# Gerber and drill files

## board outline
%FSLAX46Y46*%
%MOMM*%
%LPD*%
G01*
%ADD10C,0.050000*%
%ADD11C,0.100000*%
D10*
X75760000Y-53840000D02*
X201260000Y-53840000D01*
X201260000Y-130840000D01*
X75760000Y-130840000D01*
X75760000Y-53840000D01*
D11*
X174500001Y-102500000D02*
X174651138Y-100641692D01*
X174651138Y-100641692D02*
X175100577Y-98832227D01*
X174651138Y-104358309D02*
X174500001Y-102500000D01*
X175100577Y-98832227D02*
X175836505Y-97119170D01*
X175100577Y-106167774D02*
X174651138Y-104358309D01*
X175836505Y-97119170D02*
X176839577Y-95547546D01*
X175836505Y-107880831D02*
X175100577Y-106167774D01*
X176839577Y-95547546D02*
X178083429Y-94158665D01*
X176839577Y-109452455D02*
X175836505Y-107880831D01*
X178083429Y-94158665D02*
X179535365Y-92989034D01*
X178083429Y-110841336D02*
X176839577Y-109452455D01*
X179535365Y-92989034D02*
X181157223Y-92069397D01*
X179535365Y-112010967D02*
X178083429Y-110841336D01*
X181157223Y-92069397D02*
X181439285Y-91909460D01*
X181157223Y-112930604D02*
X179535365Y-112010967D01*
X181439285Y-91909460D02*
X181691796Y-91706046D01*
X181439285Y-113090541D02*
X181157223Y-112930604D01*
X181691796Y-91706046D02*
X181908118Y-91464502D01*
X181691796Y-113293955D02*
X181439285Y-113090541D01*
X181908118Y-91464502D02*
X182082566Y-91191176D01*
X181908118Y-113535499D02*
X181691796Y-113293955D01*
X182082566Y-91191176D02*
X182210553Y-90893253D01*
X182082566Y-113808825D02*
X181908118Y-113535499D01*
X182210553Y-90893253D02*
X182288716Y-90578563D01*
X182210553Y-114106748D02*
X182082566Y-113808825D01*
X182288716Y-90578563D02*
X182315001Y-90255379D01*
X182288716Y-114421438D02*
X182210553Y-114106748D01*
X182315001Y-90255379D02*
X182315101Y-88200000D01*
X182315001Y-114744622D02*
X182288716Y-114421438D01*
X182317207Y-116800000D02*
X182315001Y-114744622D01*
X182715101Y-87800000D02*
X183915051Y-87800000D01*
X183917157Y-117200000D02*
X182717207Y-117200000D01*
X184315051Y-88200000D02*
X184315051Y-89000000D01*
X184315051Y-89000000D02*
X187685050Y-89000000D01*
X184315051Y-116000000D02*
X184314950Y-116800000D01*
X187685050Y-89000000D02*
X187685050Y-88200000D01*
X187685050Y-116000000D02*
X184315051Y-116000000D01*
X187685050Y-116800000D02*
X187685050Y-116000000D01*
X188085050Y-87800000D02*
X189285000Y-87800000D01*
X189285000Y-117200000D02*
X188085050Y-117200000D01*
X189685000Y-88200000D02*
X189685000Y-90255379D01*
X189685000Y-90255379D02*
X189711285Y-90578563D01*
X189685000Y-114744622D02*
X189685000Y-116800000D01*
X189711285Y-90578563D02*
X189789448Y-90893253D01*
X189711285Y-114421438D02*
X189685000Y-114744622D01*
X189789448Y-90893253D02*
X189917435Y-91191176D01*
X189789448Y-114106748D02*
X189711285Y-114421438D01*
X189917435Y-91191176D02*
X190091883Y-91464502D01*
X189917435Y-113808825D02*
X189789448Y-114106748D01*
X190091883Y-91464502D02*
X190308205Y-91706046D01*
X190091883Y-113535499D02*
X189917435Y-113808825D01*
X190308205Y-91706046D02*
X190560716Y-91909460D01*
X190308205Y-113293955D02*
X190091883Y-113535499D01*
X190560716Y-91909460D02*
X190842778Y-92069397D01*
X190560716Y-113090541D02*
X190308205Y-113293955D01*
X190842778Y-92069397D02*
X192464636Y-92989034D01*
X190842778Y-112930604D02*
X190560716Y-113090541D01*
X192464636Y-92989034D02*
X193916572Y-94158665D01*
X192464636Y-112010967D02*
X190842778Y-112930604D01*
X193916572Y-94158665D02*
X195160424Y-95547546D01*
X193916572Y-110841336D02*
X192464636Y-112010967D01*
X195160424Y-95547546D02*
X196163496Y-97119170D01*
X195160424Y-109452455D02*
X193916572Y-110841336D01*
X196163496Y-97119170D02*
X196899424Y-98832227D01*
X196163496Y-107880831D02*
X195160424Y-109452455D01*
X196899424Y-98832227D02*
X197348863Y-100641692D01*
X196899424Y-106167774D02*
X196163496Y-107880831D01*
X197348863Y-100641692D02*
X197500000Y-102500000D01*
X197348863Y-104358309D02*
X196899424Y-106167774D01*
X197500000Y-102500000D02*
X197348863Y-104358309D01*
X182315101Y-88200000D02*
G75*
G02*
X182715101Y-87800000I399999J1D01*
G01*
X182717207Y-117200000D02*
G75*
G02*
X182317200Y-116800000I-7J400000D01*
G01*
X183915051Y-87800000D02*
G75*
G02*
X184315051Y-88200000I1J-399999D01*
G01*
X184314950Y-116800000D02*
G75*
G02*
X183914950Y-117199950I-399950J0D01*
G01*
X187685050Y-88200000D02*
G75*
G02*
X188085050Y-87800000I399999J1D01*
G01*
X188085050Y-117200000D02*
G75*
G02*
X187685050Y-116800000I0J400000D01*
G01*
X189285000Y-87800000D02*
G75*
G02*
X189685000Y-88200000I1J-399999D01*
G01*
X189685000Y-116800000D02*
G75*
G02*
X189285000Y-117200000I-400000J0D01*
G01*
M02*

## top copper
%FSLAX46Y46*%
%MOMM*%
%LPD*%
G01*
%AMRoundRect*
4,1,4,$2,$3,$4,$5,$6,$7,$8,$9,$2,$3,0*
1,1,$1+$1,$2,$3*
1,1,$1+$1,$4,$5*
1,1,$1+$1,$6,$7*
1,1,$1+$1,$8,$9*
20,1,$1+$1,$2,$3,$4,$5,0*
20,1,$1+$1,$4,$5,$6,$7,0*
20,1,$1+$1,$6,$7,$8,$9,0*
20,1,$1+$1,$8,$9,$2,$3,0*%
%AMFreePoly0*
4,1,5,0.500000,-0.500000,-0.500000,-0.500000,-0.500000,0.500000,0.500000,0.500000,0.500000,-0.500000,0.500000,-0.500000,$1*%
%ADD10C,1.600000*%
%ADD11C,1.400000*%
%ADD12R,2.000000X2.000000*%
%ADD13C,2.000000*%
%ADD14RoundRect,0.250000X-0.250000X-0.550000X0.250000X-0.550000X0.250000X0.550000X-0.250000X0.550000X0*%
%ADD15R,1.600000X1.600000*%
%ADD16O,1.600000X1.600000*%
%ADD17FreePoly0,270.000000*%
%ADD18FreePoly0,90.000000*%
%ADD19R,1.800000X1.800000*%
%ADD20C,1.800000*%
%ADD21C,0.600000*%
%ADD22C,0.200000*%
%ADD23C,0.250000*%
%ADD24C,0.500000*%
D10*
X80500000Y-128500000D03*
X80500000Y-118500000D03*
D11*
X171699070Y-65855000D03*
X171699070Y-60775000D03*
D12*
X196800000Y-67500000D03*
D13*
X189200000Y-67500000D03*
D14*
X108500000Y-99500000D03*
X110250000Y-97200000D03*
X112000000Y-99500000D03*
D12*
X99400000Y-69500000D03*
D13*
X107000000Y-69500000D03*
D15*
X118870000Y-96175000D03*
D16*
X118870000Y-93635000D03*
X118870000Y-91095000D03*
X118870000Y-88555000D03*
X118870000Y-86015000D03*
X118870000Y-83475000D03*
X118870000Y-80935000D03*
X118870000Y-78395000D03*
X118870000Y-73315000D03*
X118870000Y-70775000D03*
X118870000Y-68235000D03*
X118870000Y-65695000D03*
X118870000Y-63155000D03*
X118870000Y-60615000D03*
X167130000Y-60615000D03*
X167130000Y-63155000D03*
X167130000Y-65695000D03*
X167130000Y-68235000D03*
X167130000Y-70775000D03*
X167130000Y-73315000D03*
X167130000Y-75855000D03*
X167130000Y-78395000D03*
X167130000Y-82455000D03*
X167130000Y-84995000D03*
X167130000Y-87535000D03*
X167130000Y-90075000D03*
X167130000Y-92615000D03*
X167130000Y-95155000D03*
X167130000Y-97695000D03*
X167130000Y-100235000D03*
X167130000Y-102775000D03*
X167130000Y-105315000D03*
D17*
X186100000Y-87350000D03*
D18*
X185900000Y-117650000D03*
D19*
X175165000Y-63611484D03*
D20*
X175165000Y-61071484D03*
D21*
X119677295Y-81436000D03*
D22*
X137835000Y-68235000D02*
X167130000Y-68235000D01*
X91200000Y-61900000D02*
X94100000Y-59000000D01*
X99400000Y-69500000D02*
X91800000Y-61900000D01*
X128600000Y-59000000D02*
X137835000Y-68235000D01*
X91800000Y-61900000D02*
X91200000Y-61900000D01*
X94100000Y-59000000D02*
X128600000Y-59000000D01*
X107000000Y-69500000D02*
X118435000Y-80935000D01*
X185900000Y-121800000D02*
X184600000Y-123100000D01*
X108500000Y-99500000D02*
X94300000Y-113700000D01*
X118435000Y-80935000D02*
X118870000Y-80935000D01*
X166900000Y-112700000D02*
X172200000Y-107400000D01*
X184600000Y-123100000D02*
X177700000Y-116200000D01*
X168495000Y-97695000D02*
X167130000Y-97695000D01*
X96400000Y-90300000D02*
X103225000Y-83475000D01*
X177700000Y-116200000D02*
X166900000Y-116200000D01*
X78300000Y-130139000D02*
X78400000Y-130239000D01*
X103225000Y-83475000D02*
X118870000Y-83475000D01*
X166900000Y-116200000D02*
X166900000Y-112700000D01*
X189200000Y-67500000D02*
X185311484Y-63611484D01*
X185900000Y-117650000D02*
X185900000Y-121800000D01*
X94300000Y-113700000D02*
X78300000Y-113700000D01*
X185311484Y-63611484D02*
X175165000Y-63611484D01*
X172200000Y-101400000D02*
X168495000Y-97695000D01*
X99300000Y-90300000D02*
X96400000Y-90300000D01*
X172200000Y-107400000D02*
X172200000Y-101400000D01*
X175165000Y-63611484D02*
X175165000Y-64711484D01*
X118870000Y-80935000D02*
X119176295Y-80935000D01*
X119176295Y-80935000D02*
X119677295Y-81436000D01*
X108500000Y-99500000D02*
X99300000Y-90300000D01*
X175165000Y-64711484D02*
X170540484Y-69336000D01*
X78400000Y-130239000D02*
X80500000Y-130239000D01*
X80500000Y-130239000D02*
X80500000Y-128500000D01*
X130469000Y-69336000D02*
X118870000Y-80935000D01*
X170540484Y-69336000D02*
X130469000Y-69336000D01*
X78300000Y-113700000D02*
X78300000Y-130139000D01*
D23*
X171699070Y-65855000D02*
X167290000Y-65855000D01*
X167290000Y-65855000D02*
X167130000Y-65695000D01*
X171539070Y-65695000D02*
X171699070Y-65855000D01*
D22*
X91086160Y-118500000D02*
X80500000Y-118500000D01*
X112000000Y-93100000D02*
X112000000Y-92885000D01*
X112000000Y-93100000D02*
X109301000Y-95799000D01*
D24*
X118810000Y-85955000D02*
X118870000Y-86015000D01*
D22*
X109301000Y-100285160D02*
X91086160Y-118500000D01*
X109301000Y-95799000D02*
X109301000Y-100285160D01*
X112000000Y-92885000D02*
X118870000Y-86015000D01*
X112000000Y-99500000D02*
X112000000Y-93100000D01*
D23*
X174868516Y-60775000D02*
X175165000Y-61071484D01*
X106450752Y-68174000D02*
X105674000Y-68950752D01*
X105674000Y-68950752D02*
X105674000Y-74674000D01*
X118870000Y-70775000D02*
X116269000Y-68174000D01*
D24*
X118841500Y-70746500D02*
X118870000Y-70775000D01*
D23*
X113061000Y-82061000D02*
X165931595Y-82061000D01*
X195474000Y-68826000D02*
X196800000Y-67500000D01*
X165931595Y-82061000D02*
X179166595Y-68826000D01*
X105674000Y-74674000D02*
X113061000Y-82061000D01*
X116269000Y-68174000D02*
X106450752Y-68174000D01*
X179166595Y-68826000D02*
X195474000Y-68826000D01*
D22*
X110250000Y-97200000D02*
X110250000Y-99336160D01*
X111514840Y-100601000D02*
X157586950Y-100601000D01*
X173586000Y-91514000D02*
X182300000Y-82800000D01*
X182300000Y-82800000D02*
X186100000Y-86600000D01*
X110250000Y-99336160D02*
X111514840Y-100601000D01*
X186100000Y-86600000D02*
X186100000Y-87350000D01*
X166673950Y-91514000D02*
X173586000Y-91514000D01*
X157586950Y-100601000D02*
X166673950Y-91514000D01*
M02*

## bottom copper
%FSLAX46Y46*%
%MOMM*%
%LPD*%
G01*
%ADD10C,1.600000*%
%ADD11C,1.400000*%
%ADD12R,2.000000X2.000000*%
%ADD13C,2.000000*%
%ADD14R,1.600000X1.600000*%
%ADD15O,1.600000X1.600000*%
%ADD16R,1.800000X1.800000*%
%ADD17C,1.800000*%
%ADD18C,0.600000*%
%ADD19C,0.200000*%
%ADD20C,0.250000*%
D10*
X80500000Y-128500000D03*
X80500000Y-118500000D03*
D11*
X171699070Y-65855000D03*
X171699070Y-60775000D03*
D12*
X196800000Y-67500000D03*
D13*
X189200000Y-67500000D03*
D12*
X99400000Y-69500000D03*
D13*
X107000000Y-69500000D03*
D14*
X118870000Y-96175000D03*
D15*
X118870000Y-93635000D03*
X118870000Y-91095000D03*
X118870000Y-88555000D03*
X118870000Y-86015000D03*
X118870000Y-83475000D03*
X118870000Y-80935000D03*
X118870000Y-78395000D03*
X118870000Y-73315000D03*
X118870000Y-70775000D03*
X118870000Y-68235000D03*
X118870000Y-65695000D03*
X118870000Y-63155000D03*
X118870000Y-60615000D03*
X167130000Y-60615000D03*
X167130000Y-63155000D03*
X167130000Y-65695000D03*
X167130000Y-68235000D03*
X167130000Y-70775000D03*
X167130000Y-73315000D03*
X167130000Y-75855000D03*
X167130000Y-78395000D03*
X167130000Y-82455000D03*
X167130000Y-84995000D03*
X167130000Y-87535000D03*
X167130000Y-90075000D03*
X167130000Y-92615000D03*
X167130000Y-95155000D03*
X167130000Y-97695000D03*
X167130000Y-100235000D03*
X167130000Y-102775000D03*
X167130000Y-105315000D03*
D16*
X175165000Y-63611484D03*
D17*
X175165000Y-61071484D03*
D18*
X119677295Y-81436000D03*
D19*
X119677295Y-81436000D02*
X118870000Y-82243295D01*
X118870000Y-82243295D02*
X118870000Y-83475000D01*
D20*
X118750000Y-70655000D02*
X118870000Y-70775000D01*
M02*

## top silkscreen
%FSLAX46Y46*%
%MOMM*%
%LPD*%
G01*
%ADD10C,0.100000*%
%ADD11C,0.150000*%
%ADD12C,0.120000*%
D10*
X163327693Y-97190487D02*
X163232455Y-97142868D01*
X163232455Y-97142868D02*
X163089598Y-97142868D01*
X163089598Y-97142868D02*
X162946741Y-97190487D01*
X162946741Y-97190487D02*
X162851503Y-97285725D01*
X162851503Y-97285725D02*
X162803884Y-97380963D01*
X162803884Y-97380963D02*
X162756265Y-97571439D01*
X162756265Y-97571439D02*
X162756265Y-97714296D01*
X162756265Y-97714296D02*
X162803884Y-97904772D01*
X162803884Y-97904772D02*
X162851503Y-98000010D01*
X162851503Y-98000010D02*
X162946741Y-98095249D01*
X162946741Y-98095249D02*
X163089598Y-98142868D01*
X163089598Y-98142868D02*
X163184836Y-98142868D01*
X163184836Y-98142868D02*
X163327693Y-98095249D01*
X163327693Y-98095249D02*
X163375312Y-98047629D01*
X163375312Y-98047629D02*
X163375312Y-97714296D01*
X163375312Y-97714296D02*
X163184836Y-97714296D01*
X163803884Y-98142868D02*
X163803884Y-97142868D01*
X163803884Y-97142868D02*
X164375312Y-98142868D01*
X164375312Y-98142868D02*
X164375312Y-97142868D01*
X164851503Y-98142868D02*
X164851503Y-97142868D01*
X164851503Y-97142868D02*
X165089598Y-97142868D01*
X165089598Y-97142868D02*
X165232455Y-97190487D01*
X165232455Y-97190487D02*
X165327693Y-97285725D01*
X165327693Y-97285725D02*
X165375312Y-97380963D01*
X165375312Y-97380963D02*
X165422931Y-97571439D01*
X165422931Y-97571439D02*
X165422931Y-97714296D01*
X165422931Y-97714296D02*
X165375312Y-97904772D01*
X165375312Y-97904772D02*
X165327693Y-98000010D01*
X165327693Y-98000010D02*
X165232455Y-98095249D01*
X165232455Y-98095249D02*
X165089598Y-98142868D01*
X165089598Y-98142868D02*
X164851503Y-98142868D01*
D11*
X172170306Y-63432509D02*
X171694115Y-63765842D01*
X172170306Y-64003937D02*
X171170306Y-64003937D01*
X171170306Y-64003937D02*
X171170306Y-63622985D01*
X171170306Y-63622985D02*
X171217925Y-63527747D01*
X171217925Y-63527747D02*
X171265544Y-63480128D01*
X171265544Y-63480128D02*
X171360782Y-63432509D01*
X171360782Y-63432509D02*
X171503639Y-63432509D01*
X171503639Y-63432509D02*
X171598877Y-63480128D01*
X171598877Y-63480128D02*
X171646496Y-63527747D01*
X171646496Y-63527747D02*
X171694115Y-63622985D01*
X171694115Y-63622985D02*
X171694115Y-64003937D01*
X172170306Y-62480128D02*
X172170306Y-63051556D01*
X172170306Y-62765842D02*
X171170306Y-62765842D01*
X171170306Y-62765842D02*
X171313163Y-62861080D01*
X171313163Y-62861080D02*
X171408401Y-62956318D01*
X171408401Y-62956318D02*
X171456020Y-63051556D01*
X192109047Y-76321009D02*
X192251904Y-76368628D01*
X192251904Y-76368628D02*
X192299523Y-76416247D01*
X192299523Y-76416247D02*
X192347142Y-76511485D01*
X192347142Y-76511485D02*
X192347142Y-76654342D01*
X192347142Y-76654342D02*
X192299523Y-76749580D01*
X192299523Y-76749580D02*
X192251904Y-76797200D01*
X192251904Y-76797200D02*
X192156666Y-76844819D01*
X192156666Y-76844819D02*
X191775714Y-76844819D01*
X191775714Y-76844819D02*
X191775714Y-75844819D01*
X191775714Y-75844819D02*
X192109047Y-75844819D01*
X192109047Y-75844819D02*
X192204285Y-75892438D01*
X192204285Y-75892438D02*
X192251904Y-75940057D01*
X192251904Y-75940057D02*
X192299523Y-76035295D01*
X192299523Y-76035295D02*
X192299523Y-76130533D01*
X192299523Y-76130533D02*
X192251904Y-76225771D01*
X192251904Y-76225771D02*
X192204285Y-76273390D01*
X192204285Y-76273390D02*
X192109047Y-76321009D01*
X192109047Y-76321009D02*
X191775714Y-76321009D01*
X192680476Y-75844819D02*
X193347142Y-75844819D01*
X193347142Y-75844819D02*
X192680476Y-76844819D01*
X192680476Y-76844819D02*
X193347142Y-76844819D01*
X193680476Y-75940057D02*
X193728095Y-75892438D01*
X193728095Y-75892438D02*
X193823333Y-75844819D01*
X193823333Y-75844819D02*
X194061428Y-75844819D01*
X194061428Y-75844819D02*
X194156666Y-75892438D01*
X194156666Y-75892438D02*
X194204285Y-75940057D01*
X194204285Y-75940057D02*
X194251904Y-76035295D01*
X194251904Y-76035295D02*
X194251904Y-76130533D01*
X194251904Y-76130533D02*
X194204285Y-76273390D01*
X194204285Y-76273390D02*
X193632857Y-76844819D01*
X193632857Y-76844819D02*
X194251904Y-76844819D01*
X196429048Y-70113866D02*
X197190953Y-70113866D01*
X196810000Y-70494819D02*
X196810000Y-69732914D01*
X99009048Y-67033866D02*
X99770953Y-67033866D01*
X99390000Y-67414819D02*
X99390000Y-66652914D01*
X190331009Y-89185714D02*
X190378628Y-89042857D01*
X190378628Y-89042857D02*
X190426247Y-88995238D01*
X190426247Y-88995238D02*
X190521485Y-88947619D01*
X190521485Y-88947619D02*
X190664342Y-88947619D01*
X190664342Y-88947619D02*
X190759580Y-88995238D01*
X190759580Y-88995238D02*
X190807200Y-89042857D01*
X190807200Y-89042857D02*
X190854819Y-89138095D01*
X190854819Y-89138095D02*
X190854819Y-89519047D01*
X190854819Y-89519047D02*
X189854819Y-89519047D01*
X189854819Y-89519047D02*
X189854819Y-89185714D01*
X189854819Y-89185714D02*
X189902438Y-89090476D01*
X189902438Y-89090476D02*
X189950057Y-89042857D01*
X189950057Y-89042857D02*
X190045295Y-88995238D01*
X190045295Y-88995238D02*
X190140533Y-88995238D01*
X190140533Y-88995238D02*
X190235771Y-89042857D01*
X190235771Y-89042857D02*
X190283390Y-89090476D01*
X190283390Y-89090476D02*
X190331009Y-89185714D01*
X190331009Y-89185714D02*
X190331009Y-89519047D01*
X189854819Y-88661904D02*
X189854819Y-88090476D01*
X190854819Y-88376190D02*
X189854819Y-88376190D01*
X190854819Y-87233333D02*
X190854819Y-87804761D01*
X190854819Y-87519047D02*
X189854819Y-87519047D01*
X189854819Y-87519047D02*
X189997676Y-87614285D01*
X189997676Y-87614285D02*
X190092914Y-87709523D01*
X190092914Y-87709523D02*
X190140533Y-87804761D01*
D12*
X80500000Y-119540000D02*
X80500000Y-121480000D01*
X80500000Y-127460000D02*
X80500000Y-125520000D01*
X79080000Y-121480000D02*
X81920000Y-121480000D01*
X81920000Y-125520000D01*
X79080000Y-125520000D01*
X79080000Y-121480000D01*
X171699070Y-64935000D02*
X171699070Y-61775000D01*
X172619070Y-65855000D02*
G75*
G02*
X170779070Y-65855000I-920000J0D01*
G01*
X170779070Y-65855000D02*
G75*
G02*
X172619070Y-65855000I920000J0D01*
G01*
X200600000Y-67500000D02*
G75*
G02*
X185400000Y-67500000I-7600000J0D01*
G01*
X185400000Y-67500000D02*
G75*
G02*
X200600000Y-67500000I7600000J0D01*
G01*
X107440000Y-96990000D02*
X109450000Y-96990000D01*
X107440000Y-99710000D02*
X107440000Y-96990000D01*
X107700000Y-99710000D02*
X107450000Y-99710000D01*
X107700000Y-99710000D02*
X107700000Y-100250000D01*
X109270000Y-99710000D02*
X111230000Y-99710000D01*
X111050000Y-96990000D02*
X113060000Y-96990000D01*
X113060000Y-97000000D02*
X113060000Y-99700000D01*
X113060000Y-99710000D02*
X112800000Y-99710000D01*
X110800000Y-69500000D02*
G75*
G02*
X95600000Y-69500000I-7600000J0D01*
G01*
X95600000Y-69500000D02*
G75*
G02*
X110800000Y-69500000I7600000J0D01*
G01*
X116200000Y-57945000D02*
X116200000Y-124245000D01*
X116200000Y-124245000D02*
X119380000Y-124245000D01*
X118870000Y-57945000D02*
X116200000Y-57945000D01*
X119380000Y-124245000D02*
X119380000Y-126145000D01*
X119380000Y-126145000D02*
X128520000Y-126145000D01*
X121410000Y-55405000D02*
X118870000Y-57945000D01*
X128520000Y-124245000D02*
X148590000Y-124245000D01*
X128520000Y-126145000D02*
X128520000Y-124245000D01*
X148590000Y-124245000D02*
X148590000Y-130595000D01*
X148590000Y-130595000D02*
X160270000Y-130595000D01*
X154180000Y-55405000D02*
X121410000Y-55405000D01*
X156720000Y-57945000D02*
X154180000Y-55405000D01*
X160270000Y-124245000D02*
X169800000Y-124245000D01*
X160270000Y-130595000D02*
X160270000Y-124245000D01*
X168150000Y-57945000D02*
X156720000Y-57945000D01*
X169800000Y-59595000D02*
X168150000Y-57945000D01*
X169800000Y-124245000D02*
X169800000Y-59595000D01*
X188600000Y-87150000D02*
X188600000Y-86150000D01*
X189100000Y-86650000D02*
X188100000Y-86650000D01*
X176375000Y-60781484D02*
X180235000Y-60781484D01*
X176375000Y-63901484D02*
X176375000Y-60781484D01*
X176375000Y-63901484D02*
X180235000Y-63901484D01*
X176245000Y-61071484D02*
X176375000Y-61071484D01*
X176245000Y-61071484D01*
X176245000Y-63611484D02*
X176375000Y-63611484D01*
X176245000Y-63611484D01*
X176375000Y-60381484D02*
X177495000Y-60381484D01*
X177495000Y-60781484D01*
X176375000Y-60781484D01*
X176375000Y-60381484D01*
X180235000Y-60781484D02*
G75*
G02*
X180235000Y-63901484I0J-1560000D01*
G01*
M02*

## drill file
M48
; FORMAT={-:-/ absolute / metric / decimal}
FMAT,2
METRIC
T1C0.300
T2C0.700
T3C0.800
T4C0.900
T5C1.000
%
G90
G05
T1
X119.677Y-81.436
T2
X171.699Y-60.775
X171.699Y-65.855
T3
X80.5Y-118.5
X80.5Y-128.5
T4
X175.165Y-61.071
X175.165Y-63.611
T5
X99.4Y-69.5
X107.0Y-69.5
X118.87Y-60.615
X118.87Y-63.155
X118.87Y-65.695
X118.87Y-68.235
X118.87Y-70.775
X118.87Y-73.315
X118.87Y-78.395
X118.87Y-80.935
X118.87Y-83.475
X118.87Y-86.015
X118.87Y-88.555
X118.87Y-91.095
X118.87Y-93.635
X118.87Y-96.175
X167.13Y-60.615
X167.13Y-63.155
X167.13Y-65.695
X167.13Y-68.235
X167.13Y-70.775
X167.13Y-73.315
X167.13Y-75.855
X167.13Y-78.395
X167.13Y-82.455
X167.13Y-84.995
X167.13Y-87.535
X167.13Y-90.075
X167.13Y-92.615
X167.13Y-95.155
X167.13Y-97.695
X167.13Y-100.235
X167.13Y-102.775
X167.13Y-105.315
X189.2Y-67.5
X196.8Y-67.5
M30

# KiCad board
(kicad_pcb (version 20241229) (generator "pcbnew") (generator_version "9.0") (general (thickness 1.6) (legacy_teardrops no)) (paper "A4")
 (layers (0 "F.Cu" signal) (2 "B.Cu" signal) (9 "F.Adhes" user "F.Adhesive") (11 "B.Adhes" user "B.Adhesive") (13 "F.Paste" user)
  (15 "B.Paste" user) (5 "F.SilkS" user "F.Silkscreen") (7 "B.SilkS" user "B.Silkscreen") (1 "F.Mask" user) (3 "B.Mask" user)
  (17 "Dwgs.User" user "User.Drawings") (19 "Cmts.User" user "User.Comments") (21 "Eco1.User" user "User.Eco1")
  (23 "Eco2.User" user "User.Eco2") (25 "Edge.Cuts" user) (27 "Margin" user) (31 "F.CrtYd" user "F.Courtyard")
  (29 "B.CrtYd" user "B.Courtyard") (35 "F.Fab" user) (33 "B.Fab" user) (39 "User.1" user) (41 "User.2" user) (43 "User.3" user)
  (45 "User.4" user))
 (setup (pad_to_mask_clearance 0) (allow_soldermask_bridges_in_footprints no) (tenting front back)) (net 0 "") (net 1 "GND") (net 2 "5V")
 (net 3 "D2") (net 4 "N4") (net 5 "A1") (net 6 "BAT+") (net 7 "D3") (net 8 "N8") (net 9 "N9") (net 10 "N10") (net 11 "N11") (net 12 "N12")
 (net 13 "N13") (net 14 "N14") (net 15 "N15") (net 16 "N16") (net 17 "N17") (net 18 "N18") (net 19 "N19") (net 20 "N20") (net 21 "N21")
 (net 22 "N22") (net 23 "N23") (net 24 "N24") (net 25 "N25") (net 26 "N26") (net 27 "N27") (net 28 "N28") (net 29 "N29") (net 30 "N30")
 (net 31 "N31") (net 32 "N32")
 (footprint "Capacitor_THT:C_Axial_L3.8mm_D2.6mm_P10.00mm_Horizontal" (layer "F.Cu") (at 80.5 128.5 90)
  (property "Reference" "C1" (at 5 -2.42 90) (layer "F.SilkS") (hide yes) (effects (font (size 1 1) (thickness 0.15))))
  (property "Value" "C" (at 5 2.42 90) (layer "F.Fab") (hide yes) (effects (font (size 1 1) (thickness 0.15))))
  (fp_line (start 8.96 0) (end 7.02 0) (stroke (width 0.12) (type solid)) (layer "F.SilkS"))
  (fp_line (start 1.04 0) (end 2.98 0) (stroke (width 0.12) (type solid)) (layer "F.SilkS"))
  (fp_rect (start 2.98 -1.42) (end 7.02 1.42) (stroke (width 0.12) (type solid)) (fill no) (layer "F.SilkS"))
  (pad "1" thru_hole circle (at 0 0 90) (size 1.6 1.6) (drill 0.8) (layers "*.Cu" "*.Mask") (remove_unused_layers no) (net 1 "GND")
   (zone_connect 1))
  (pad "2" thru_hole circle (at 10 0 90) (size 1.6 1.6) (drill 0.8) (layers "*.Cu" "*.Mask") (remove_unused_layers no) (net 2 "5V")))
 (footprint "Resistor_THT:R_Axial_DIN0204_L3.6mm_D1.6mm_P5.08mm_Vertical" (layer "F.Cu") (at 171.69907 65.855 90)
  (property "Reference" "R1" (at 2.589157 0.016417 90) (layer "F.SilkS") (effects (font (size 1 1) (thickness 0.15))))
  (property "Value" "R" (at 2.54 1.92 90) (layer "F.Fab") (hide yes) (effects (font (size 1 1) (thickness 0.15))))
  (fp_line (start 0.92 0) (end 4.08 0) (stroke (width 0.12) (type solid)) (layer "F.SilkS"))
  (fp_circle (center 0 0) (end 0.92 0) (stroke (width 0.12) (type solid)) (fill no) (layer "F.SilkS"))
  (pad "1" thru_hole circle (at 0 0 90) (size 1.4 1.4) (drill 0.7) (layers "*.Cu" "*.Mask") (remove_unused_layers no) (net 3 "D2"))
  (pad "2" thru_hole circle (at 5.08 0 90) (size 1.4 1.4) (drill 0.7) (layers "*.Cu" "*.Mask") (remove_unused_layers no) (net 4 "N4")))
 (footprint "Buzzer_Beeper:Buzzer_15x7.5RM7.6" (layer "F.Cu") (at 196.8 67.5 180)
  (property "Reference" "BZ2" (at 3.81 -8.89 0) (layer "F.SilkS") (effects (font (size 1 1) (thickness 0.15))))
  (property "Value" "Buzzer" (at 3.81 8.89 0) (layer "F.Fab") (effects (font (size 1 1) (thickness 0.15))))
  (fp_circle (center 3.8 0) (end 11.4 0) (stroke (width 0.12) (type solid)) (fill no) (layer "F.SilkS"))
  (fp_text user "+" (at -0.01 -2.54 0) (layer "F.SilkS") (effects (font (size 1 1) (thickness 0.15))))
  (pad "1" thru_hole rect (at 0 0 180) (size 2 2) (drill 1) (layers "*.Cu" "*.Mask") (remove_unused_layers no) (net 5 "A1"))
  (pad "2" thru_hole circle (at 7.6 0 180) (size 2 2) (drill 1) (layers "*.Cu" "*.Mask") (remove_unused_layers no) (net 1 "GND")))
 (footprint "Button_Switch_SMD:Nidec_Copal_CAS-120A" (layer "F.Cu") (at 110.25 98.35 90)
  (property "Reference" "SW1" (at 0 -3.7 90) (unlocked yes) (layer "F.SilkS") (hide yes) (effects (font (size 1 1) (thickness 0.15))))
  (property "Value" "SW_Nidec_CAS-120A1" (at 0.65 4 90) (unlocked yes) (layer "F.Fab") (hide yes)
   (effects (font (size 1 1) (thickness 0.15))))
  (fp_line (start 1.36 -2.81) (end 1.36 -0.8) (stroke (width 0.12) (type solid)) (layer "F.SilkS"))
  (fp_line (start -1.36 -2.81) (end 1.36 -2.81) (stroke (width 0.12) (type solid)) (layer "F.SilkS"))
  (fp_line (start -1.36 -2.55) (end -1.36 -2.8) (stroke (width 0.12) (type solid)) (layer "F.SilkS"))
  (fp_line (start -1.36 -2.55) (end -1.9 -2.55) (stroke (width 0.12) (type default)) (layer "F.SilkS"))
  (fp_line (start -1.36 -0.98) (end -1.36 0.98) (stroke (width 0.12) (type solid)) (layer "F.SilkS"))
  (fp_line (start 1.36 0.8) (end 1.36 2.81) (stroke (width 0.12) (type solid)) (layer "F.SilkS"))
  (fp_line (start 1.35 2.81) (end -1.35 2.81) (stroke (width 0.12) (type solid)) (layer "F.SilkS"))
  (fp_line (start -1.36 2.81) (end -1.36 2.55) (stroke (width 0.12) (type solid)) (layer "F.SilkS"))
  (pad "1" smd roundrect (at -1.15 -1.75) (size 1 1.6) (layers "F.Cu" "F.Mask" "F.Paste") (roundrect_rratio 0.25) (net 1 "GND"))
  (pad "2" smd roundrect (at 1.15 0) (size 1 1.6) (layers "F.Cu" "F.Mask" "F.Paste") (roundrect_rratio 0.25) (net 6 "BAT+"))
  (pad "3" smd roundrect (at -1.15 1.75) (size 1 1.6) (layers "F.Cu" "F.Mask" "F.Paste") (roundrect_rratio 0.25) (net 2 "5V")))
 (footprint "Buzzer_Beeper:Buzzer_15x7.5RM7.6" (layer "F.Cu") (at 99.4 69.5)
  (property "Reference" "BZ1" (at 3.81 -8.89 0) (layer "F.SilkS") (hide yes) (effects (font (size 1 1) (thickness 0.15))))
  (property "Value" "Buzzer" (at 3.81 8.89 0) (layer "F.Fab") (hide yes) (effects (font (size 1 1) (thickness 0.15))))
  (fp_circle (center 3.8 0) (end 11.4 0) (stroke (width 0.12) (type solid)) (fill no) (layer "F.SilkS"))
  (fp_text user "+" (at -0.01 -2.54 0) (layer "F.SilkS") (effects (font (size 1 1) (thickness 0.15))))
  (pad "1" thru_hole rect (at 0 0) (size 2 2) (drill 1) (layers "*.Cu" "*.Mask") (remove_unused_layers no) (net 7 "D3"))
  (pad "2" thru_hole circle (at 7.6 0) (size 2 2) (drill 1) (layers "*.Cu" "*.Mask") (remove_unused_layers no) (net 1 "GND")))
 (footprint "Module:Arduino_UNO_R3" (layer "F.Cu") (at 118.87 96.175 90)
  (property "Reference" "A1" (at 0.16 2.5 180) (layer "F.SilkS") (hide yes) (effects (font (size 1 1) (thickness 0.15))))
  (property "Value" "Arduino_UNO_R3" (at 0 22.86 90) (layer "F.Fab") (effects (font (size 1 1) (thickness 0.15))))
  (fp_line (start 38.23 -2.67) (end -28.07 -2.67) (stroke (width 0.12) (type solid)) (layer "F.SilkS"))
  (fp_line (start -28.07 -2.67) (end -28.07 0.51) (stroke (width 0.12) (type solid)) (layer "F.SilkS"))
  (fp_line (start 38.23 0) (end 38.23 -2.67) (stroke (width 0.12) (type solid)) (layer "F.SilkS"))
  (fp_line (start -28.07 0.51) (end -29.97 0.51) (stroke (width 0.12) (type solid)) (layer "F.SilkS"))
  (fp_line (start -29.97 0.51) (end -29.97 9.65) (stroke (width 0.12) (type solid)) (layer "F.SilkS"))
  (fp_line (start 40.77 2.54) (end 38.23 0) (stroke (width 0.12) (type solid)) (layer "F.SilkS"))
  (fp_line (start -28.07 9.65) (end -28.07 29.72) (stroke (width 0.12) (type solid)) (layer "F.SilkS"))
  (fp_line (start -29.97 9.65) (end -28.07 9.65) (stroke (width 0.12) (type solid)) (layer "F.SilkS"))
  (fp_line (start -28.07 29.72) (end -34.42 29.72) (stroke (width 0.12) (type solid)) (layer "F.SilkS"))
  (fp_line (start -34.42 29.72) (end -34.42 41.4) (stroke (width 0.12) (type solid)) (layer "F.SilkS"))
  (fp_line (start 40.77 35.31) (end 40.77 2.54) (stroke (width 0.12) (type solid)) (layer "F.SilkS"))
  (fp_line (start 38.23 37.85) (end 40.77 35.31) (stroke (width 0.12) (type solid)) (layer "F.SilkS"))
  (fp_line (start -28.07 41.4) (end -28.07 50.93) (stroke (width 0.12) (type solid)) (layer "F.SilkS"))
  (fp_line (start -34.42 41.4) (end -28.07 41.4) (stroke (width 0.12) (type solid)) (layer "F.SilkS"))
  (fp_line (start 38.23 49.28) (end 38.23 37.85) (stroke (width 0.12) (type solid)) (layer "F.SilkS"))
  (fp_line (start 36.58 50.93) (end 38.23 49.28) (stroke (width 0.12) (type solid)) (layer "F.SilkS"))
  (fp_line (start -28.07 50.93) (end 36.58 50.93) (stroke (width 0.12) (type solid)) (layer "F.SilkS"))
  (pad "1" thru_hole rect (at 0 0 180) (size 1.6 1.6) (drill 1) (layers "*.Cu" "*.Mask") (remove_unused_layers no) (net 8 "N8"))
  (pad "2" thru_hole oval (at 2.54 0 180) (size 1.6 1.6) (drill 1) (layers "*.Cu" "*.Mask") (remove_unused_layers no) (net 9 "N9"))
  (pad "3" thru_hole oval (at 5.08 0 180) (size 1.6 1.6) (drill 1) (layers "*.Cu" "*.Mask") (remove_unused_layers no) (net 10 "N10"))
  (pad "4" thru_hole oval (at 7.62 0 180) (size 1.6 1.6) (drill 1) (layers "*.Cu" "*.Mask") (remove_unused_layers no) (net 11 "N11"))
  (pad "5" thru_hole oval (at 10.16 0 180) (size 1.6 1.6) (drill 1) (layers "*.Cu" "*.Mask") (remove_unused_layers no) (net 2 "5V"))
  (pad "6" thru_hole oval (at 12.7 0 180) (size 1.6 1.6) (drill 1) (layers "*.Cu" "*.Mask") (remove_unused_layers no) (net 1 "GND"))
  (pad "7" thru_hole oval (at 15.24 0 180) (size 1.6 1.6) (drill 1) (layers "*.Cu" "*.Mask") (remove_unused_layers no) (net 1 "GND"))
  (pad "8" thru_hole oval (at 17.78 0 180) (size 1.6 1.6) (drill 1) (layers "*.Cu" "*.Mask") (remove_unused_layers no) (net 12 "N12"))
  (pad "9" thru_hole oval (at 22.86 0 180) (size 1.6 1.6) (drill 1) (layers "*.Cu" "*.Mask") (remove_unused_layers no) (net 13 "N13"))
  (pad "10" thru_hole oval (at 25.4 0 180) (size 1.6 1.6) (drill 1) (layers "*.Cu" "*.Mask") (remove_unused_layers no) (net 5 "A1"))
  (pad "11" thru_hole oval (at 27.94 0 180) (size 1.6 1.6) (drill 1) (layers "*.Cu" "*.Mask") (remove_unused_layers no) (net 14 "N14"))
  (pad "12" thru_hole oval (at 30.48 0 180) (size 1.6 1.6) (drill 1) (layers "*.Cu" "*.Mask") (remove_unused_layers no) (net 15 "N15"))
  (pad "13" thru_hole oval (at 33.02 0 180) (size 1.6 1.6) (drill 1) (layers "*.Cu" "*.Mask") (remove_unused_layers no) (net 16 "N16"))
  (pad "14" thru_hole oval (at 35.56 0 180) (size 1.6 1.6) (drill 1) (layers "*.Cu" "*.Mask") (remove_unused_layers no) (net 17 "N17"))
  (pad "15" thru_hole oval (at 35.56 48.26 180) (size 1.6 1.6) (drill 1) (layers "*.Cu" "*.Mask") (remove_unused_layers no) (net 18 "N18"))
  (pad "16" thru_hole oval (at 33.02 48.26 180) (size 1.6 1.6) (drill 1) (layers "*.Cu" "*.Mask") (remove_unused_layers no) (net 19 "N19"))
  (pad "17" thru_hole oval (at 30.48 48.26 180) (size 1.6 1.6) (drill 1) (layers "*.Cu" "*.Mask") (remove_unused_layers no) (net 3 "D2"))
  (pad "18" thru_hole oval (at 27.94 48.26 180) (size 1.6 1.6) (drill 1) (layers "*.Cu" "*.Mask") (remove_unused_layers no) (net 7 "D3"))
  (pad "19" thru_hole oval (at 25.4 48.26 180) (size 1.6 1.6) (drill 1) (layers "*.Cu" "*.Mask") (remove_unused_layers no) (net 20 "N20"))
  (pad "20" thru_hole oval (at 22.86 48.26 180) (size 1.6 1.6) (drill 1) (layers "*.Cu" "*.Mask") (remove_unused_layers no) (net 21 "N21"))
  (pad "21" thru_hole oval (at 20.32 48.26 180) (size 1.6 1.6) (drill 1) (layers "*.Cu" "*.Mask") (remove_unused_layers no) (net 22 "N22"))
  (pad "22" thru_hole oval (at 17.78 48.26 180) (size 1.6 1.6) (drill 1) (layers "*.Cu" "*.Mask") (remove_unused_layers no) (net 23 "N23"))
  (pad "23" thru_hole oval (at 13.72 48.26 180) (size 1.6 1.6) (drill 1) (layers "*.Cu" "*.Mask") (remove_unused_layers no) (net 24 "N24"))
  (pad "24" thru_hole oval (at 11.18 48.26 180) (size 1.6 1.6) (drill 1) (layers "*.Cu" "*.Mask") (remove_unused_layers no) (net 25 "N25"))
  (pad "25" thru_hole oval (at 8.64 48.26 180) (size 1.6 1.6) (drill 1) (layers "*.Cu" "*.Mask") (remove_unused_layers no) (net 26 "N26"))
  (pad "26" thru_hole oval (at 6.1 48.26 180) (size 1.6 1.6) (drill 1) (layers "*.Cu" "*.Mask") (remove_unused_layers no) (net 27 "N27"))
  (pad "27" thru_hole oval (at 3.56 48.26 180) (size 1.6 1.6) (drill 1) (layers "*.Cu" "*.Mask") (remove_unused_layers no) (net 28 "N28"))
  (pad "28" thru_hole oval (at 1.02 48.26 180) (size 1.6 1.6) (drill 1) (layers "*.Cu" "*.Mask") (remove_unused_layers no) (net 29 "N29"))
  (pad "29" thru_hole oval (at -1.52 48.26 180) (size 1.6 1.6) (drill 1) (layers "*.Cu" "*.Mask") (remove_unused_layers no) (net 1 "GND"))
  (pad "30" thru_hole oval (at -4.06 48.26 180) (size 1.6 1.6) (drill 1) (layers "*.Cu" "*.Mask") (remove_unused_layers no) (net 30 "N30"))
  (pad "31" thru_hole oval (at -6.6 48.26 180) (size 1.6 1.6) (drill 1) (layers "*.Cu" "*.Mask") (remove_unused_layers no) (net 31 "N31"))
  (pad "32" thru_hole oval (at -9.14 48.26 180) (size 1.6 1.6) (drill 1) (layers "*.Cu" "*.Mask") (remove_unused_layers no) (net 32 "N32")))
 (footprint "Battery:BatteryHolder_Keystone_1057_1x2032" (layer "F.Cu") (at 186 102.5 -90)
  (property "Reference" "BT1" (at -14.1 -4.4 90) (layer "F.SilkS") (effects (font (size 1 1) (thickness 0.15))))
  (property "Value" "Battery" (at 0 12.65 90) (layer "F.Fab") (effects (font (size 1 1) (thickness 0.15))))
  (fp_line (start -15.35 -2.6) (end -16.35 -2.6) (stroke (width 0.12) (type solid)) (layer "F.SilkS"))
  (fp_line (start -15.85 -3.1) (end -15.85 -2.1) (stroke (width 0.12) (type solid)) (layer "F.SilkS"))
  (fp_line (start 0 11.499999) (end -1.858308 11.348862) (stroke (width 0.1) (type solid)) (layer "Edge.Cuts"))
  (fp_line (start -1.858308 11.348862) (end -3.667773 10.899423) (stroke (width 0.1) (type solid)) (layer "Edge.Cuts"))
  (fp_line (start 1.858309 11.348862) (end 0 11.499999) (stroke (width 0.1) (type solid)) (layer "Edge.Cuts"))
  (fp_line (start -3.667773 10.899423) (end -5.38083 10.163495) (stroke (width 0.1) (type solid)) (layer "Edge.Cuts"))
  (fp_line (start 3.667774 10.899423) (end 1.858309 11.348862) (stroke (width 0.1) (type solid)) (layer "Edge.Cuts"))
  (fp_line (start -5.38083 10.163495) (end -6.952454 9.160423) (stroke (width 0.1) (type solid)) (layer "Edge.Cuts"))
  (fp_line (start 5.380831 10.163495) (end 3.667774 10.899423) (stroke (width 0.1) (type solid)) (layer "Edge.Cuts"))
  (fp_line (start -6.952454 9.160423) (end -8.341335 7.916571) (stroke (width 0.1) (type solid)) (layer "Edge.Cuts"))
  (fp_line (start 6.952455 9.160423) (end 5.380831 10.163495) (stroke (width 0.1) (type solid)) (layer "Edge.Cuts"))
  (fp_line (start -8.341335 7.916571) (end -9.510966 6.464635) (stroke (width 0.1) (type solid)) (layer "Edge.Cuts"))
  (fp_line (start 8.341336 7.916571) (end 6.952455 9.160423) (stroke (width 0.1) (type solid)) (layer "Edge.Cuts"))
  (fp_line (start -9.510966 6.464635) (end -10.430603 4.842777) (stroke (width 0.1) (type solid)) (layer "Edge.Cuts"))
  (fp_line (start 9.510967 6.464635) (end 8.341336 7.916571) (stroke (width 0.1) (type solid)) (layer "Edge.Cuts"))
  (fp_line (start -10.430603 4.842777) (end -10.59054 4.560715) (stroke (width 0.1) (type solid)) (layer "Edge.Cuts"))
  (fp_line (start 10.430604 4.842777) (end 9.510967 6.464635) (stroke (width 0.1) (type solid)) (layer "Edge.Cuts"))
  (fp_line (start -10.59054 4.560715) (end -10.793954 4.308204) (stroke (width 0.1) (type solid)) (layer "Edge.Cuts"))
  (fp_line (start 10.590541 4.560715) (end 10.430604 4.842777) (stroke (width 0.1) (type solid)) (layer "Edge.Cuts"))
  (fp_line (start -10.793954 4.308204) (end -11.035498 4.091882) (stroke (width 0.1) (type solid)) (layer "Edge.Cuts"))
  (fp_line (start 10.793955 4.308204) (end 10.590541 4.560715) (stroke (width 0.1) (type solid)) (layer "Edge.Cuts"))
  (fp_line (start -11.035498 4.091882) (end -11.308824 3.917434) (stroke (width 0.1) (type solid)) (layer "Edge.Cuts"))
  (fp_line (start 11.035499 4.091882) (end 10.793955 4.308204) (stroke (width 0.1) (type solid)) (layer "Edge.Cuts"))
  (fp_line (start -11.308824 3.917434) (end -11.606747 3.789447) (stroke (width 0.1) (type solid)) (layer "Edge.Cuts"))
  (fp_line (start 11.308825 3.917434) (end 11.035499 4.091882) (stroke (width 0.1) (type solid)) (layer "Edge.Cuts"))
  (fp_line (start -11.606747 3.789447) (end -11.921437 3.711284) (stroke (width 0.1) (type solid)) (layer "Edge.Cuts"))
  (fp_line (start 11.606748 3.789447) (end 11.308825 3.917434) (stroke (width 0.1) (type solid)) (layer "Edge.Cuts"))
  (fp_line (start -11.921437 3.711284) (end -12.244621 3.684999) (stroke (width 0.1) (type solid)) (layer "Edge.Cuts"))
  (fp_line (start 11.921438 3.711284) (end 11.606748 3.789447) (stroke (width 0.1) (type solid)) (layer "Edge.Cuts"))
  (fp_line (start -12.244621 3.684999) (end -14.3 3.684899) (stroke (width 0.1) (type solid)) (layer "Edge.Cuts"))
  (fp_line (start 12.244622 3.684999) (end 11.921438 3.711284) (stroke (width 0.1) (type solid)) (layer "Edge.Cuts"))
  (fp_line (start 14.3 3.682793) (end 12.244622 3.684999) (stroke (width 0.1) (type solid)) (layer "Edge.Cuts"))
  (fp_line (start -14.7 3.284899) (end -14.7 2.084949) (stroke (width 0.1) (type solid)) (layer "Edge.Cuts"))
  (fp_line (start 14.7 2.082843) (end 14.7 3.282793) (stroke (width 0.1) (type solid)) (layer "Edge.Cuts"))
  (fp_line (start -14.3 1.684949) (end -13.5 1.684949) (stroke (width 0.1) (type solid)) (layer "Edge.Cuts"))
  (fp_line (start -13.5 1.684949) (end -13.5 -1.68505) (stroke (width 0.1) (type solid)) (layer "Edge.Cuts"))
  (fp_line (start 13.5 1.684949) (end 14.3 1.68505) (stroke (width 0.1) (type solid)) (layer "Edge.Cuts"))
  (fp_line (start -13.5 -1.68505) (end -14.3 -1.68505) (stroke (width 0.1) (type solid)) (layer "Edge.Cuts"))
  (fp_line (start 13.5 -1.68505) (end 13.5 1.684949) (stroke (width 0.1) (type solid)) (layer "Edge.Cuts"))
  (fp_line (start 14.3 -1.68505) (end 13.5 -1.68505) (stroke (width 0.1) (type solid)) (layer "Edge.Cuts"))
  (fp_line (start -14.7 -2.08505) (end -14.7 -3.285) (stroke (width 0.1) (type solid)) (layer "Edge.Cuts"))
  (fp_line (start 14.7 -3.285) (end 14.7 -2.08505) (stroke (width 0.1) (type solid)) (layer "Edge.Cuts"))
  (fp_line (start -14.3 -3.685) (end -12.244621 -3.685) (stroke (width 0.1) (type solid)) (layer "Edge.Cuts"))
  (fp_line (start -12.244621 -3.685) (end -11.921437 -3.711285) (stroke (width 0.1) (type solid)) (layer "Edge.Cuts"))
  (fp_line (start 12.244622 -3.685) (end 14.3 -3.685) (stroke (width 0.1) (type solid)) (layer "Edge.Cuts"))
  (fp_line (start -11.921437 -3.711285) (end -11.606747 -3.789448) (stroke (width 0.1) (type solid)) (layer "Edge.Cuts"))
  (fp_line (start 11.921438 -3.711285) (end 12.244622 -3.685) (stroke (width 0.1) (type solid)) (layer "Edge.Cuts"))
  (fp_line (start -11.606747 -3.789448) (end -11.308824 -3.917435) (stroke (width 0.1) (type solid)) (layer "Edge.Cuts"))
  (fp_line (start 11.606748 -3.789448) (end 11.921438 -3.711285) (stroke (width 0.1) (type solid)) (layer "Edge.Cuts"))
  (fp_line (start -11.308824 -3.917435) (end -11.035498 -4.091883) (stroke (width 0.1) (type solid)) (layer "Edge.Cuts"))
  (fp_line (start 11.308825 -3.917435) (end 11.606748 -3.789448) (stroke (width 0.1) (type solid)) (layer "Edge.Cuts"))
  (fp_line (start -11.035498 -4.091883) (end -10.793954 -4.308205) (stroke (width 0.1) (type solid)) (layer "Edge.Cuts"))
  (fp_line (start 11.035499 -4.091883) (end 11.308825 -3.917435) (stroke (width 0.1) (type solid)) (layer "Edge.Cuts"))
  (fp_line (start -10.793954 -4.308205) (end -10.59054 -4.560716) (stroke (width 0.1) (type solid)) (layer "Edge.Cuts"))
  (fp_line (start 10.793955 -4.308205) (end 11.035499 -4.091883) (stroke (width 0.1) (type solid)) (layer "Edge.Cuts"))
  (fp_line (start -10.59054 -4.560716) (end -10.430603 -4.842778) (stroke (width 0.1) (type solid)) (layer "Edge.Cuts"))
  (fp_line (start 10.590541 -4.560716) (end 10.793955 -4.308205) (stroke (width 0.1) (type solid)) (layer "Edge.Cuts"))
  (fp_line (start -10.430603 -4.842778) (end -9.510966 -6.464636) (stroke (width 0.1) (type solid)) (layer "Edge.Cuts"))
  (fp_line (start 10.430604 -4.842778) (end 10.590541 -4.560716) (stroke (width 0.1) (type solid)) (layer "Edge.Cuts"))
  (fp_line (start -9.510966 -6.464636) (end -8.341335 -7.916572) (stroke (width 0.1) (type solid)) (layer "Edge.Cuts"))
  (fp_line (start 9.510967 -6.464636) (end 10.430604 -4.842778) (stroke (width 0.1) (type solid)) (layer "Edge.Cuts"))
  (fp_line (start -8.341335 -7.916572) (end -6.952454 -9.160424) (stroke (width 0.1) (type solid)) (layer "Edge.Cuts"))
  (fp_line (start 8.341336 -7.916572) (end 9.510967 -6.464636) (stroke (width 0.1) (type solid)) (layer "Edge.Cuts"))
  (fp_line (start -6.952454 -9.160424) (end -5.38083 -10.163496) (stroke (width 0.1) (type solid)) (layer "Edge.Cuts"))
  (fp_line (start 6.952455 -9.160424) (end 8.341336 -7.916572) (stroke (width 0.1) (type solid)) (layer "Edge.Cuts"))
  (fp_line (start -5.38083 -10.163496) (end -3.667773 -10.899424) (stroke (width 0.1) (type solid)) (layer "Edge.Cuts"))
  (fp_line (start 5.380831 -10.163496) (end 6.952455 -9.160424) (stroke (width 0.1) (type solid)) (layer "Edge.Cuts"))
  (fp_line (start -3.667773 -10.899424) (end -1.858308 -11.348863) (stroke (width 0.1) (type solid)) (layer "Edge.Cuts"))
  (fp_line (start 3.667774 -10.899424) (end 5.380831 -10.163496) (stroke (width 0.1) (type solid)) (layer "Edge.Cuts"))
  (fp_line (start -1.858308 -11.348863) (end 0 -11.5) (stroke (width 0.1) (type solid)) (layer "Edge.Cuts"))
  (fp_line (start 1.858309 -11.348863) (end 3.667774 -10.899424) (stroke (width 0.1) (type solid)) (layer "Edge.Cuts"))
  (fp_line (start 0 -11.5) (end 1.858309 -11.348863) (stroke (width 0.1) (type solid)) (layer "Edge.Cuts"))
  (fp_arc (start -14.3 3.684899) (mid -14.582843 3.567742) (end -14.7 3.284899) (stroke (width 0.1) (type solid)) (layer "Edge.Cuts"))
  (fp_arc (start 14.7 3.282793) (mid 14.582843 3.565636) (end 14.3 3.682793) (stroke (width 0.1) (type solid)) (layer "Edge.Cuts"))
  (fp_arc (start -14.7 2.084949) (mid -14.582843 1.802106) (end -14.3 1.684949) (stroke (width 0.1) (type solid)) (layer "Edge.Cuts"))
  (fp_arc (start 14.3 1.68505) (mid 14.582843 1.802207) (end 14.7 2.08505) (stroke (width 0.1) (type solid)) (layer "Edge.Cuts"))
  (fp_arc (start -14.3 -1.68505) (mid -14.582843 -1.802207) (end -14.7 -2.08505) (stroke (width 0.1) (type solid)) (layer "Edge.Cuts"))
  (fp_arc (start 14.7 -2.08505) (mid 14.582843 -1.802207) (end 14.3 -1.68505) (stroke (width 0.1) (type solid)) (layer "Edge.Cuts"))
  (fp_arc (start -14.7 -3.285) (mid -14.582843 -3.567843) (end -14.3 -3.685) (stroke (width 0.1) (type solid)) (layer "Edge.Cuts"))
  (fp_arc (start 14.3 -3.685) (mid 14.582843 -3.567843) (end 14.7 -3.285) (stroke (width 0.1) (type solid)) (layer "Edge.Cuts"))
  (pad "1" smd custom (at -15.15 -0.1 270) (size 1 1) (layers "F.Cu" "F.Mask" "F.Paste") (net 6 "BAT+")
   (options (clearance outline) (anchor rect)) (primitives))
  (pad "2" smd custom (at 15.15 0.1 90) (size 1 1) (layers "F.Cu" "F.Mask" "F.Paste") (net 1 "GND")
   (options (clearance outline) (anchor rect)) (primitives)))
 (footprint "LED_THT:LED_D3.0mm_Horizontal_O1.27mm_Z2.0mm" (layer "F.Cu") (at 175.165 63.611484 90)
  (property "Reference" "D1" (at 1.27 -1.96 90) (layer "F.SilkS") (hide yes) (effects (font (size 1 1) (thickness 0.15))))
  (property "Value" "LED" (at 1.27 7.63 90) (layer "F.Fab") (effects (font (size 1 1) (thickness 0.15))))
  (fp_line (start 2.83 1.21) (end 2.83 5.07) (stroke (width 0.12) (type solid)) (layer "F.SilkS"))
  (fp_line (start -0.29 1.21) (end 2.83 1.21) (stroke (width 0.12) (type solid)) (layer "F.SilkS"))
  (fp_line (start -0.29 1.21) (end -0.29 5.07) (stroke (width 0.12) (type solid)) (layer "F.SilkS"))
  (fp_rect (start 2.54 1.08) (end 2.54 1.21) (stroke (width 0.12) (type solid)) (fill no) (layer "F.SilkS"))
  (fp_rect (start 0 1.08) (end 0 1.21) (stroke (width 0.12) (type solid)) (fill no) (layer "F.SilkS"))
  (fp_rect (start 2.83 1.21) (end 3.23 2.33) (stroke (width 0.12) (type solid)) (fill no) (layer "F.SilkS"))
  (fp_arc (start 2.83 5.07) (mid 1.27 6.63) (end -0.29 5.07) (stroke (width 0.12) (type solid)) (layer "F.SilkS"))
  (pad "1" thru_hole rect (at 0 0 90) (size 1.8 1.8) (drill 0.9) (layers "*.Cu" "*.Mask") (remove_unused_layers no) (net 1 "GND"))
  (pad "2" thru_hole circle (at 2.54 0 90) (size 1.8 1.8) (drill 0.9) (layers "*.Cu" "*.Mask") (remove_unused_layers no) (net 4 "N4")))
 (gr_rect (start 75.76 53.84) (end 201.26 130.84) (stroke (width 0.05) (type default)) (fill no) (layer "Edge.Cuts"))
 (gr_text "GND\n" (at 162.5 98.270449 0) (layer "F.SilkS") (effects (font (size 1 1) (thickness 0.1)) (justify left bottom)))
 (segment (start 137.835 68.235) (end 167.13 68.235) (width 0.2) (layer "F.Cu") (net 7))
 (segment (start 91.2 61.9) (end 94.1 59) (width 0.2) (layer "F.Cu") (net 7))
 (segment (start 99.4 69.5) (end 91.8 61.9) (width 0.2) (layer "F.Cu") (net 7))
 (segment (start 128.6 59) (end 137.835 68.235) (width 0.2) (layer "F.Cu") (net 7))
 (segment (start 91.8 61.9) (end 91.2 61.9) (width 0.2) (layer "F.Cu") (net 7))
 (segment (start 94.1 59) (end 128.6 59) (width 0.2) (layer "F.Cu") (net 7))
 (segment (start 107 69.5) (end 118.435 80.935) (width 0.2) (layer "F.Cu") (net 1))
 (segment (start 185.9 121.8) (end 184.6 123.1) (width 0.2) (layer "F.Cu") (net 1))
 (segment (start 108.5 99.5) (end 94.3 113.7) (width 0.2) (layer "F.Cu") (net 1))
 (segment (start 118.435 80.935) (end 118.87 80.935) (width 0.2) (layer "F.Cu") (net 1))
 (segment (start 166.9 112.7) (end 172.2 107.4) (width 0.2) (layer "F.Cu") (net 1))
 (segment (start 184.6 123.1) (end 177.7 116.2) (width 0.2) (layer "F.Cu") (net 1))
 (segment (start 168.495 97.695) (end 167.13 97.695) (width 0.2) (layer "F.Cu") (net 1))
 (segment (start 96.4 90.3) (end 103.225 83.475) (width 0.2) (layer "F.Cu") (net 1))
 (segment (start 177.7 116.2) (end 166.9 116.2) (width 0.2) (layer "F.Cu") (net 1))
 (segment (start 78.3 130.139) (end 78.4 130.239) (width 0.2) (layer "F.Cu") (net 1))
 (segment (start 103.225 83.475) (end 118.87 83.475) (width 0.2) (layer "F.Cu") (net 1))
 (segment (start 166.9 116.2) (end 166.9 112.7) (width 0.2) (layer "F.Cu") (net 1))
 (segment (start 189.2 67.5) (end 185.311484 63.611484) (width 0.2) (layer "F.Cu") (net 1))
 (segment (start 185.9 117.65) (end 185.9 121.8) (width 0.2) (layer "F.Cu") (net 1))
 (segment (start 94.3 113.7) (end 78.3 113.7) (width 0.2) (layer "F.Cu") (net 1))
 (segment (start 185.311484 63.611484) (end 175.165 63.611484) (width 0.2) (layer "F.Cu") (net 1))
 (segment (start 172.2 101.4) (end 168.495 97.695) (width 0.2) (layer "F.Cu") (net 1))
 (segment (start 99.3 90.3) (end 96.4 90.3) (width 0.2) (layer "F.Cu") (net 1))
 (segment (start 172.2 107.4) (end 172.2 101.4) (width 0.2) (layer "F.Cu") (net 1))
 (segment (start 175.165 63.611484) (end 175.165 64.711484) (width 0.2) (layer "F.Cu") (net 1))
 (segment (start 118.87 80.935) (end 119.176295 80.935) (width 0.2) (layer "F.Cu") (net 1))
 (segment (start 119.176295 80.935) (end 119.677295 81.436) (width 0.2) (layer "F.Cu") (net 1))
 (segment (start 108.5 99.5) (end 99.3 90.3) (width 0.2) (layer "F.Cu") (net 1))
 (segment (start 175.165 64.711484) (end 170.540484 69.336) (width 0.2) (layer "F.Cu") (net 1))
 (segment (start 78.4 130.239) (end 80.5 130.239) (width 0.2) (layer "F.Cu") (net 1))
 (segment (start 80.5 130.239) (end 80.5 128.5) (width 0.2) (layer "F.Cu") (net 1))
 (segment (start 130.469 69.336) (end 118.87 80.935) (width 0.2) (layer "F.Cu") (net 1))
 (segment (start 170.540484 69.336) (end 130.469 69.336) (width 0.2) (layer "F.Cu") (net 1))
 (segment (start 78.3 113.7) (end 78.3 130.139) (width 0.2) (layer "F.Cu") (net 1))
 (via (at 119.677295 81.436) (size 0.6) (drill 0.3) (layers "F.Cu" "B.Cu") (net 1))
 (segment (start 119.677295 81.436) (end 118.87 82.243295) (width 0.2) (layer "B.Cu") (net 1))
 (segment (start 118.87 82.243295) (end 118.87 83.475) (width 0.2) (layer "B.Cu") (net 1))
 (segment (start 171.69907 65.855) (end 167.29 65.855) (width 0.25) (layer "F.Cu") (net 3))
 (segment (start 167.29 65.855) (end 167.13 65.695) (width 0.25) (layer "F.Cu") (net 3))
 (segment (start 171.53907 65.695) (end 171.69907 65.855) (width 0.25) (layer "F.Cu") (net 3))
 (segment (start 91.08616 118.5) (end 80.5 118.5) (width 0.2) (layer "F.Cu") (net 2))
 (segment (start 112 93.1) (end 112 92.885) (width 0.2) (layer "F.Cu") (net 2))
 (segment (start 112 93.1) (end 109.301 95.799) (width 0.2) (layer "F.Cu") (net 2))
 (segment (start 118.81 85.955) (end 118.87 86.015) (width 0.5) (layer "F.Cu") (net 2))
 (segment (start 109.301 100.28516) (end 91.08616 118.5) (width 0.2) (layer "F.Cu") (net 2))
 (segment (start 109.301 95.799) (end 109.301 100.28516) (width 0.2) (layer "F.Cu") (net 2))
 (segment (start 112 92.885) (end 118.87 86.015) (width 0.2) (layer "F.Cu") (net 2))
 (segment (start 112 99.5) (end 112 93.1) (width 0.2) (layer "F.Cu") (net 2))
 (segment (start 174.868516 60.775) (end 175.165 61.071484) (width 0.25) (layer "F.Cu") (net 4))
 (segment (start 106.450752 68.174) (end 105.674 68.950752) (width 0.25) (layer "F.Cu") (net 5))
 (segment (start 105.674 68.950752) (end 105.674 74.674) (width 0.25) (layer "F.Cu") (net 5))
 (segment (start 118.87 70.775) (end 116.269 68.174) (width 0.25) (layer "F.Cu") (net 5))
 (segment (start 118.8415 70.7465) (end 118.87 70.775) (width 0.5) (layer "F.Cu") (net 5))
 (segment (start 113.061 82.061) (end 165.931595 82.061) (width 0.25) (layer "F.Cu") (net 5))
 (segment (start 195.474 68.826) (end 196.8 67.5) (width 0.25) (layer "F.Cu") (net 5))
 (segment (start 165.931595 82.061) (end 179.166595 68.826) (width 0.25) (layer "F.Cu") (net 5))
 (segment (start 105.674 74.674) (end 113.061 82.061) (width 0.25) (layer "F.Cu") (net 5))
 (segment (start 116.269 68.174) (end 106.450752 68.174) (width 0.25) (layer "F.Cu") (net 5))
 (segment (start 179.166595 68.826) (end 195.474 68.826) (width 0.25) (layer "F.Cu") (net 5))
 (segment (start 118.75 70.655) (end 118.87 70.775) (width 0.25) (layer "B.Cu") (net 5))
 (segment (start 110.25 97.2) (end 110.25 99.33616) (width 0.2) (layer "F.Cu") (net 6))
 (segment (start 111.51484 100.601) (end 157.58695 100.601) (width 0.2) (layer "F.Cu") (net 6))
 (segment (start 173.586 91.514) (end 182.3 82.8) (width 0.2) (layer "F.Cu") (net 6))
 (segment (start 182.3 82.8) (end 186.1 86.6) (width 0.2) (layer "F.Cu") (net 6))
 (segment (start 110.25 99.33616) (end 111.51484 100.601) (width 0.2) (layer "F.Cu") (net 6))
 (segment (start 186.1 86.6) (end 186.1 87.35) (width 0.2) (layer "F.Cu") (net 6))
 (segment (start 166.67395 91.514) (end 173.586 91.514) (width 0.2) (layer "F.Cu") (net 6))
 (segment (start 157.58695 100.601) (end 166.67395 91.514) (width 0.2) (layer "F.Cu") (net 6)))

